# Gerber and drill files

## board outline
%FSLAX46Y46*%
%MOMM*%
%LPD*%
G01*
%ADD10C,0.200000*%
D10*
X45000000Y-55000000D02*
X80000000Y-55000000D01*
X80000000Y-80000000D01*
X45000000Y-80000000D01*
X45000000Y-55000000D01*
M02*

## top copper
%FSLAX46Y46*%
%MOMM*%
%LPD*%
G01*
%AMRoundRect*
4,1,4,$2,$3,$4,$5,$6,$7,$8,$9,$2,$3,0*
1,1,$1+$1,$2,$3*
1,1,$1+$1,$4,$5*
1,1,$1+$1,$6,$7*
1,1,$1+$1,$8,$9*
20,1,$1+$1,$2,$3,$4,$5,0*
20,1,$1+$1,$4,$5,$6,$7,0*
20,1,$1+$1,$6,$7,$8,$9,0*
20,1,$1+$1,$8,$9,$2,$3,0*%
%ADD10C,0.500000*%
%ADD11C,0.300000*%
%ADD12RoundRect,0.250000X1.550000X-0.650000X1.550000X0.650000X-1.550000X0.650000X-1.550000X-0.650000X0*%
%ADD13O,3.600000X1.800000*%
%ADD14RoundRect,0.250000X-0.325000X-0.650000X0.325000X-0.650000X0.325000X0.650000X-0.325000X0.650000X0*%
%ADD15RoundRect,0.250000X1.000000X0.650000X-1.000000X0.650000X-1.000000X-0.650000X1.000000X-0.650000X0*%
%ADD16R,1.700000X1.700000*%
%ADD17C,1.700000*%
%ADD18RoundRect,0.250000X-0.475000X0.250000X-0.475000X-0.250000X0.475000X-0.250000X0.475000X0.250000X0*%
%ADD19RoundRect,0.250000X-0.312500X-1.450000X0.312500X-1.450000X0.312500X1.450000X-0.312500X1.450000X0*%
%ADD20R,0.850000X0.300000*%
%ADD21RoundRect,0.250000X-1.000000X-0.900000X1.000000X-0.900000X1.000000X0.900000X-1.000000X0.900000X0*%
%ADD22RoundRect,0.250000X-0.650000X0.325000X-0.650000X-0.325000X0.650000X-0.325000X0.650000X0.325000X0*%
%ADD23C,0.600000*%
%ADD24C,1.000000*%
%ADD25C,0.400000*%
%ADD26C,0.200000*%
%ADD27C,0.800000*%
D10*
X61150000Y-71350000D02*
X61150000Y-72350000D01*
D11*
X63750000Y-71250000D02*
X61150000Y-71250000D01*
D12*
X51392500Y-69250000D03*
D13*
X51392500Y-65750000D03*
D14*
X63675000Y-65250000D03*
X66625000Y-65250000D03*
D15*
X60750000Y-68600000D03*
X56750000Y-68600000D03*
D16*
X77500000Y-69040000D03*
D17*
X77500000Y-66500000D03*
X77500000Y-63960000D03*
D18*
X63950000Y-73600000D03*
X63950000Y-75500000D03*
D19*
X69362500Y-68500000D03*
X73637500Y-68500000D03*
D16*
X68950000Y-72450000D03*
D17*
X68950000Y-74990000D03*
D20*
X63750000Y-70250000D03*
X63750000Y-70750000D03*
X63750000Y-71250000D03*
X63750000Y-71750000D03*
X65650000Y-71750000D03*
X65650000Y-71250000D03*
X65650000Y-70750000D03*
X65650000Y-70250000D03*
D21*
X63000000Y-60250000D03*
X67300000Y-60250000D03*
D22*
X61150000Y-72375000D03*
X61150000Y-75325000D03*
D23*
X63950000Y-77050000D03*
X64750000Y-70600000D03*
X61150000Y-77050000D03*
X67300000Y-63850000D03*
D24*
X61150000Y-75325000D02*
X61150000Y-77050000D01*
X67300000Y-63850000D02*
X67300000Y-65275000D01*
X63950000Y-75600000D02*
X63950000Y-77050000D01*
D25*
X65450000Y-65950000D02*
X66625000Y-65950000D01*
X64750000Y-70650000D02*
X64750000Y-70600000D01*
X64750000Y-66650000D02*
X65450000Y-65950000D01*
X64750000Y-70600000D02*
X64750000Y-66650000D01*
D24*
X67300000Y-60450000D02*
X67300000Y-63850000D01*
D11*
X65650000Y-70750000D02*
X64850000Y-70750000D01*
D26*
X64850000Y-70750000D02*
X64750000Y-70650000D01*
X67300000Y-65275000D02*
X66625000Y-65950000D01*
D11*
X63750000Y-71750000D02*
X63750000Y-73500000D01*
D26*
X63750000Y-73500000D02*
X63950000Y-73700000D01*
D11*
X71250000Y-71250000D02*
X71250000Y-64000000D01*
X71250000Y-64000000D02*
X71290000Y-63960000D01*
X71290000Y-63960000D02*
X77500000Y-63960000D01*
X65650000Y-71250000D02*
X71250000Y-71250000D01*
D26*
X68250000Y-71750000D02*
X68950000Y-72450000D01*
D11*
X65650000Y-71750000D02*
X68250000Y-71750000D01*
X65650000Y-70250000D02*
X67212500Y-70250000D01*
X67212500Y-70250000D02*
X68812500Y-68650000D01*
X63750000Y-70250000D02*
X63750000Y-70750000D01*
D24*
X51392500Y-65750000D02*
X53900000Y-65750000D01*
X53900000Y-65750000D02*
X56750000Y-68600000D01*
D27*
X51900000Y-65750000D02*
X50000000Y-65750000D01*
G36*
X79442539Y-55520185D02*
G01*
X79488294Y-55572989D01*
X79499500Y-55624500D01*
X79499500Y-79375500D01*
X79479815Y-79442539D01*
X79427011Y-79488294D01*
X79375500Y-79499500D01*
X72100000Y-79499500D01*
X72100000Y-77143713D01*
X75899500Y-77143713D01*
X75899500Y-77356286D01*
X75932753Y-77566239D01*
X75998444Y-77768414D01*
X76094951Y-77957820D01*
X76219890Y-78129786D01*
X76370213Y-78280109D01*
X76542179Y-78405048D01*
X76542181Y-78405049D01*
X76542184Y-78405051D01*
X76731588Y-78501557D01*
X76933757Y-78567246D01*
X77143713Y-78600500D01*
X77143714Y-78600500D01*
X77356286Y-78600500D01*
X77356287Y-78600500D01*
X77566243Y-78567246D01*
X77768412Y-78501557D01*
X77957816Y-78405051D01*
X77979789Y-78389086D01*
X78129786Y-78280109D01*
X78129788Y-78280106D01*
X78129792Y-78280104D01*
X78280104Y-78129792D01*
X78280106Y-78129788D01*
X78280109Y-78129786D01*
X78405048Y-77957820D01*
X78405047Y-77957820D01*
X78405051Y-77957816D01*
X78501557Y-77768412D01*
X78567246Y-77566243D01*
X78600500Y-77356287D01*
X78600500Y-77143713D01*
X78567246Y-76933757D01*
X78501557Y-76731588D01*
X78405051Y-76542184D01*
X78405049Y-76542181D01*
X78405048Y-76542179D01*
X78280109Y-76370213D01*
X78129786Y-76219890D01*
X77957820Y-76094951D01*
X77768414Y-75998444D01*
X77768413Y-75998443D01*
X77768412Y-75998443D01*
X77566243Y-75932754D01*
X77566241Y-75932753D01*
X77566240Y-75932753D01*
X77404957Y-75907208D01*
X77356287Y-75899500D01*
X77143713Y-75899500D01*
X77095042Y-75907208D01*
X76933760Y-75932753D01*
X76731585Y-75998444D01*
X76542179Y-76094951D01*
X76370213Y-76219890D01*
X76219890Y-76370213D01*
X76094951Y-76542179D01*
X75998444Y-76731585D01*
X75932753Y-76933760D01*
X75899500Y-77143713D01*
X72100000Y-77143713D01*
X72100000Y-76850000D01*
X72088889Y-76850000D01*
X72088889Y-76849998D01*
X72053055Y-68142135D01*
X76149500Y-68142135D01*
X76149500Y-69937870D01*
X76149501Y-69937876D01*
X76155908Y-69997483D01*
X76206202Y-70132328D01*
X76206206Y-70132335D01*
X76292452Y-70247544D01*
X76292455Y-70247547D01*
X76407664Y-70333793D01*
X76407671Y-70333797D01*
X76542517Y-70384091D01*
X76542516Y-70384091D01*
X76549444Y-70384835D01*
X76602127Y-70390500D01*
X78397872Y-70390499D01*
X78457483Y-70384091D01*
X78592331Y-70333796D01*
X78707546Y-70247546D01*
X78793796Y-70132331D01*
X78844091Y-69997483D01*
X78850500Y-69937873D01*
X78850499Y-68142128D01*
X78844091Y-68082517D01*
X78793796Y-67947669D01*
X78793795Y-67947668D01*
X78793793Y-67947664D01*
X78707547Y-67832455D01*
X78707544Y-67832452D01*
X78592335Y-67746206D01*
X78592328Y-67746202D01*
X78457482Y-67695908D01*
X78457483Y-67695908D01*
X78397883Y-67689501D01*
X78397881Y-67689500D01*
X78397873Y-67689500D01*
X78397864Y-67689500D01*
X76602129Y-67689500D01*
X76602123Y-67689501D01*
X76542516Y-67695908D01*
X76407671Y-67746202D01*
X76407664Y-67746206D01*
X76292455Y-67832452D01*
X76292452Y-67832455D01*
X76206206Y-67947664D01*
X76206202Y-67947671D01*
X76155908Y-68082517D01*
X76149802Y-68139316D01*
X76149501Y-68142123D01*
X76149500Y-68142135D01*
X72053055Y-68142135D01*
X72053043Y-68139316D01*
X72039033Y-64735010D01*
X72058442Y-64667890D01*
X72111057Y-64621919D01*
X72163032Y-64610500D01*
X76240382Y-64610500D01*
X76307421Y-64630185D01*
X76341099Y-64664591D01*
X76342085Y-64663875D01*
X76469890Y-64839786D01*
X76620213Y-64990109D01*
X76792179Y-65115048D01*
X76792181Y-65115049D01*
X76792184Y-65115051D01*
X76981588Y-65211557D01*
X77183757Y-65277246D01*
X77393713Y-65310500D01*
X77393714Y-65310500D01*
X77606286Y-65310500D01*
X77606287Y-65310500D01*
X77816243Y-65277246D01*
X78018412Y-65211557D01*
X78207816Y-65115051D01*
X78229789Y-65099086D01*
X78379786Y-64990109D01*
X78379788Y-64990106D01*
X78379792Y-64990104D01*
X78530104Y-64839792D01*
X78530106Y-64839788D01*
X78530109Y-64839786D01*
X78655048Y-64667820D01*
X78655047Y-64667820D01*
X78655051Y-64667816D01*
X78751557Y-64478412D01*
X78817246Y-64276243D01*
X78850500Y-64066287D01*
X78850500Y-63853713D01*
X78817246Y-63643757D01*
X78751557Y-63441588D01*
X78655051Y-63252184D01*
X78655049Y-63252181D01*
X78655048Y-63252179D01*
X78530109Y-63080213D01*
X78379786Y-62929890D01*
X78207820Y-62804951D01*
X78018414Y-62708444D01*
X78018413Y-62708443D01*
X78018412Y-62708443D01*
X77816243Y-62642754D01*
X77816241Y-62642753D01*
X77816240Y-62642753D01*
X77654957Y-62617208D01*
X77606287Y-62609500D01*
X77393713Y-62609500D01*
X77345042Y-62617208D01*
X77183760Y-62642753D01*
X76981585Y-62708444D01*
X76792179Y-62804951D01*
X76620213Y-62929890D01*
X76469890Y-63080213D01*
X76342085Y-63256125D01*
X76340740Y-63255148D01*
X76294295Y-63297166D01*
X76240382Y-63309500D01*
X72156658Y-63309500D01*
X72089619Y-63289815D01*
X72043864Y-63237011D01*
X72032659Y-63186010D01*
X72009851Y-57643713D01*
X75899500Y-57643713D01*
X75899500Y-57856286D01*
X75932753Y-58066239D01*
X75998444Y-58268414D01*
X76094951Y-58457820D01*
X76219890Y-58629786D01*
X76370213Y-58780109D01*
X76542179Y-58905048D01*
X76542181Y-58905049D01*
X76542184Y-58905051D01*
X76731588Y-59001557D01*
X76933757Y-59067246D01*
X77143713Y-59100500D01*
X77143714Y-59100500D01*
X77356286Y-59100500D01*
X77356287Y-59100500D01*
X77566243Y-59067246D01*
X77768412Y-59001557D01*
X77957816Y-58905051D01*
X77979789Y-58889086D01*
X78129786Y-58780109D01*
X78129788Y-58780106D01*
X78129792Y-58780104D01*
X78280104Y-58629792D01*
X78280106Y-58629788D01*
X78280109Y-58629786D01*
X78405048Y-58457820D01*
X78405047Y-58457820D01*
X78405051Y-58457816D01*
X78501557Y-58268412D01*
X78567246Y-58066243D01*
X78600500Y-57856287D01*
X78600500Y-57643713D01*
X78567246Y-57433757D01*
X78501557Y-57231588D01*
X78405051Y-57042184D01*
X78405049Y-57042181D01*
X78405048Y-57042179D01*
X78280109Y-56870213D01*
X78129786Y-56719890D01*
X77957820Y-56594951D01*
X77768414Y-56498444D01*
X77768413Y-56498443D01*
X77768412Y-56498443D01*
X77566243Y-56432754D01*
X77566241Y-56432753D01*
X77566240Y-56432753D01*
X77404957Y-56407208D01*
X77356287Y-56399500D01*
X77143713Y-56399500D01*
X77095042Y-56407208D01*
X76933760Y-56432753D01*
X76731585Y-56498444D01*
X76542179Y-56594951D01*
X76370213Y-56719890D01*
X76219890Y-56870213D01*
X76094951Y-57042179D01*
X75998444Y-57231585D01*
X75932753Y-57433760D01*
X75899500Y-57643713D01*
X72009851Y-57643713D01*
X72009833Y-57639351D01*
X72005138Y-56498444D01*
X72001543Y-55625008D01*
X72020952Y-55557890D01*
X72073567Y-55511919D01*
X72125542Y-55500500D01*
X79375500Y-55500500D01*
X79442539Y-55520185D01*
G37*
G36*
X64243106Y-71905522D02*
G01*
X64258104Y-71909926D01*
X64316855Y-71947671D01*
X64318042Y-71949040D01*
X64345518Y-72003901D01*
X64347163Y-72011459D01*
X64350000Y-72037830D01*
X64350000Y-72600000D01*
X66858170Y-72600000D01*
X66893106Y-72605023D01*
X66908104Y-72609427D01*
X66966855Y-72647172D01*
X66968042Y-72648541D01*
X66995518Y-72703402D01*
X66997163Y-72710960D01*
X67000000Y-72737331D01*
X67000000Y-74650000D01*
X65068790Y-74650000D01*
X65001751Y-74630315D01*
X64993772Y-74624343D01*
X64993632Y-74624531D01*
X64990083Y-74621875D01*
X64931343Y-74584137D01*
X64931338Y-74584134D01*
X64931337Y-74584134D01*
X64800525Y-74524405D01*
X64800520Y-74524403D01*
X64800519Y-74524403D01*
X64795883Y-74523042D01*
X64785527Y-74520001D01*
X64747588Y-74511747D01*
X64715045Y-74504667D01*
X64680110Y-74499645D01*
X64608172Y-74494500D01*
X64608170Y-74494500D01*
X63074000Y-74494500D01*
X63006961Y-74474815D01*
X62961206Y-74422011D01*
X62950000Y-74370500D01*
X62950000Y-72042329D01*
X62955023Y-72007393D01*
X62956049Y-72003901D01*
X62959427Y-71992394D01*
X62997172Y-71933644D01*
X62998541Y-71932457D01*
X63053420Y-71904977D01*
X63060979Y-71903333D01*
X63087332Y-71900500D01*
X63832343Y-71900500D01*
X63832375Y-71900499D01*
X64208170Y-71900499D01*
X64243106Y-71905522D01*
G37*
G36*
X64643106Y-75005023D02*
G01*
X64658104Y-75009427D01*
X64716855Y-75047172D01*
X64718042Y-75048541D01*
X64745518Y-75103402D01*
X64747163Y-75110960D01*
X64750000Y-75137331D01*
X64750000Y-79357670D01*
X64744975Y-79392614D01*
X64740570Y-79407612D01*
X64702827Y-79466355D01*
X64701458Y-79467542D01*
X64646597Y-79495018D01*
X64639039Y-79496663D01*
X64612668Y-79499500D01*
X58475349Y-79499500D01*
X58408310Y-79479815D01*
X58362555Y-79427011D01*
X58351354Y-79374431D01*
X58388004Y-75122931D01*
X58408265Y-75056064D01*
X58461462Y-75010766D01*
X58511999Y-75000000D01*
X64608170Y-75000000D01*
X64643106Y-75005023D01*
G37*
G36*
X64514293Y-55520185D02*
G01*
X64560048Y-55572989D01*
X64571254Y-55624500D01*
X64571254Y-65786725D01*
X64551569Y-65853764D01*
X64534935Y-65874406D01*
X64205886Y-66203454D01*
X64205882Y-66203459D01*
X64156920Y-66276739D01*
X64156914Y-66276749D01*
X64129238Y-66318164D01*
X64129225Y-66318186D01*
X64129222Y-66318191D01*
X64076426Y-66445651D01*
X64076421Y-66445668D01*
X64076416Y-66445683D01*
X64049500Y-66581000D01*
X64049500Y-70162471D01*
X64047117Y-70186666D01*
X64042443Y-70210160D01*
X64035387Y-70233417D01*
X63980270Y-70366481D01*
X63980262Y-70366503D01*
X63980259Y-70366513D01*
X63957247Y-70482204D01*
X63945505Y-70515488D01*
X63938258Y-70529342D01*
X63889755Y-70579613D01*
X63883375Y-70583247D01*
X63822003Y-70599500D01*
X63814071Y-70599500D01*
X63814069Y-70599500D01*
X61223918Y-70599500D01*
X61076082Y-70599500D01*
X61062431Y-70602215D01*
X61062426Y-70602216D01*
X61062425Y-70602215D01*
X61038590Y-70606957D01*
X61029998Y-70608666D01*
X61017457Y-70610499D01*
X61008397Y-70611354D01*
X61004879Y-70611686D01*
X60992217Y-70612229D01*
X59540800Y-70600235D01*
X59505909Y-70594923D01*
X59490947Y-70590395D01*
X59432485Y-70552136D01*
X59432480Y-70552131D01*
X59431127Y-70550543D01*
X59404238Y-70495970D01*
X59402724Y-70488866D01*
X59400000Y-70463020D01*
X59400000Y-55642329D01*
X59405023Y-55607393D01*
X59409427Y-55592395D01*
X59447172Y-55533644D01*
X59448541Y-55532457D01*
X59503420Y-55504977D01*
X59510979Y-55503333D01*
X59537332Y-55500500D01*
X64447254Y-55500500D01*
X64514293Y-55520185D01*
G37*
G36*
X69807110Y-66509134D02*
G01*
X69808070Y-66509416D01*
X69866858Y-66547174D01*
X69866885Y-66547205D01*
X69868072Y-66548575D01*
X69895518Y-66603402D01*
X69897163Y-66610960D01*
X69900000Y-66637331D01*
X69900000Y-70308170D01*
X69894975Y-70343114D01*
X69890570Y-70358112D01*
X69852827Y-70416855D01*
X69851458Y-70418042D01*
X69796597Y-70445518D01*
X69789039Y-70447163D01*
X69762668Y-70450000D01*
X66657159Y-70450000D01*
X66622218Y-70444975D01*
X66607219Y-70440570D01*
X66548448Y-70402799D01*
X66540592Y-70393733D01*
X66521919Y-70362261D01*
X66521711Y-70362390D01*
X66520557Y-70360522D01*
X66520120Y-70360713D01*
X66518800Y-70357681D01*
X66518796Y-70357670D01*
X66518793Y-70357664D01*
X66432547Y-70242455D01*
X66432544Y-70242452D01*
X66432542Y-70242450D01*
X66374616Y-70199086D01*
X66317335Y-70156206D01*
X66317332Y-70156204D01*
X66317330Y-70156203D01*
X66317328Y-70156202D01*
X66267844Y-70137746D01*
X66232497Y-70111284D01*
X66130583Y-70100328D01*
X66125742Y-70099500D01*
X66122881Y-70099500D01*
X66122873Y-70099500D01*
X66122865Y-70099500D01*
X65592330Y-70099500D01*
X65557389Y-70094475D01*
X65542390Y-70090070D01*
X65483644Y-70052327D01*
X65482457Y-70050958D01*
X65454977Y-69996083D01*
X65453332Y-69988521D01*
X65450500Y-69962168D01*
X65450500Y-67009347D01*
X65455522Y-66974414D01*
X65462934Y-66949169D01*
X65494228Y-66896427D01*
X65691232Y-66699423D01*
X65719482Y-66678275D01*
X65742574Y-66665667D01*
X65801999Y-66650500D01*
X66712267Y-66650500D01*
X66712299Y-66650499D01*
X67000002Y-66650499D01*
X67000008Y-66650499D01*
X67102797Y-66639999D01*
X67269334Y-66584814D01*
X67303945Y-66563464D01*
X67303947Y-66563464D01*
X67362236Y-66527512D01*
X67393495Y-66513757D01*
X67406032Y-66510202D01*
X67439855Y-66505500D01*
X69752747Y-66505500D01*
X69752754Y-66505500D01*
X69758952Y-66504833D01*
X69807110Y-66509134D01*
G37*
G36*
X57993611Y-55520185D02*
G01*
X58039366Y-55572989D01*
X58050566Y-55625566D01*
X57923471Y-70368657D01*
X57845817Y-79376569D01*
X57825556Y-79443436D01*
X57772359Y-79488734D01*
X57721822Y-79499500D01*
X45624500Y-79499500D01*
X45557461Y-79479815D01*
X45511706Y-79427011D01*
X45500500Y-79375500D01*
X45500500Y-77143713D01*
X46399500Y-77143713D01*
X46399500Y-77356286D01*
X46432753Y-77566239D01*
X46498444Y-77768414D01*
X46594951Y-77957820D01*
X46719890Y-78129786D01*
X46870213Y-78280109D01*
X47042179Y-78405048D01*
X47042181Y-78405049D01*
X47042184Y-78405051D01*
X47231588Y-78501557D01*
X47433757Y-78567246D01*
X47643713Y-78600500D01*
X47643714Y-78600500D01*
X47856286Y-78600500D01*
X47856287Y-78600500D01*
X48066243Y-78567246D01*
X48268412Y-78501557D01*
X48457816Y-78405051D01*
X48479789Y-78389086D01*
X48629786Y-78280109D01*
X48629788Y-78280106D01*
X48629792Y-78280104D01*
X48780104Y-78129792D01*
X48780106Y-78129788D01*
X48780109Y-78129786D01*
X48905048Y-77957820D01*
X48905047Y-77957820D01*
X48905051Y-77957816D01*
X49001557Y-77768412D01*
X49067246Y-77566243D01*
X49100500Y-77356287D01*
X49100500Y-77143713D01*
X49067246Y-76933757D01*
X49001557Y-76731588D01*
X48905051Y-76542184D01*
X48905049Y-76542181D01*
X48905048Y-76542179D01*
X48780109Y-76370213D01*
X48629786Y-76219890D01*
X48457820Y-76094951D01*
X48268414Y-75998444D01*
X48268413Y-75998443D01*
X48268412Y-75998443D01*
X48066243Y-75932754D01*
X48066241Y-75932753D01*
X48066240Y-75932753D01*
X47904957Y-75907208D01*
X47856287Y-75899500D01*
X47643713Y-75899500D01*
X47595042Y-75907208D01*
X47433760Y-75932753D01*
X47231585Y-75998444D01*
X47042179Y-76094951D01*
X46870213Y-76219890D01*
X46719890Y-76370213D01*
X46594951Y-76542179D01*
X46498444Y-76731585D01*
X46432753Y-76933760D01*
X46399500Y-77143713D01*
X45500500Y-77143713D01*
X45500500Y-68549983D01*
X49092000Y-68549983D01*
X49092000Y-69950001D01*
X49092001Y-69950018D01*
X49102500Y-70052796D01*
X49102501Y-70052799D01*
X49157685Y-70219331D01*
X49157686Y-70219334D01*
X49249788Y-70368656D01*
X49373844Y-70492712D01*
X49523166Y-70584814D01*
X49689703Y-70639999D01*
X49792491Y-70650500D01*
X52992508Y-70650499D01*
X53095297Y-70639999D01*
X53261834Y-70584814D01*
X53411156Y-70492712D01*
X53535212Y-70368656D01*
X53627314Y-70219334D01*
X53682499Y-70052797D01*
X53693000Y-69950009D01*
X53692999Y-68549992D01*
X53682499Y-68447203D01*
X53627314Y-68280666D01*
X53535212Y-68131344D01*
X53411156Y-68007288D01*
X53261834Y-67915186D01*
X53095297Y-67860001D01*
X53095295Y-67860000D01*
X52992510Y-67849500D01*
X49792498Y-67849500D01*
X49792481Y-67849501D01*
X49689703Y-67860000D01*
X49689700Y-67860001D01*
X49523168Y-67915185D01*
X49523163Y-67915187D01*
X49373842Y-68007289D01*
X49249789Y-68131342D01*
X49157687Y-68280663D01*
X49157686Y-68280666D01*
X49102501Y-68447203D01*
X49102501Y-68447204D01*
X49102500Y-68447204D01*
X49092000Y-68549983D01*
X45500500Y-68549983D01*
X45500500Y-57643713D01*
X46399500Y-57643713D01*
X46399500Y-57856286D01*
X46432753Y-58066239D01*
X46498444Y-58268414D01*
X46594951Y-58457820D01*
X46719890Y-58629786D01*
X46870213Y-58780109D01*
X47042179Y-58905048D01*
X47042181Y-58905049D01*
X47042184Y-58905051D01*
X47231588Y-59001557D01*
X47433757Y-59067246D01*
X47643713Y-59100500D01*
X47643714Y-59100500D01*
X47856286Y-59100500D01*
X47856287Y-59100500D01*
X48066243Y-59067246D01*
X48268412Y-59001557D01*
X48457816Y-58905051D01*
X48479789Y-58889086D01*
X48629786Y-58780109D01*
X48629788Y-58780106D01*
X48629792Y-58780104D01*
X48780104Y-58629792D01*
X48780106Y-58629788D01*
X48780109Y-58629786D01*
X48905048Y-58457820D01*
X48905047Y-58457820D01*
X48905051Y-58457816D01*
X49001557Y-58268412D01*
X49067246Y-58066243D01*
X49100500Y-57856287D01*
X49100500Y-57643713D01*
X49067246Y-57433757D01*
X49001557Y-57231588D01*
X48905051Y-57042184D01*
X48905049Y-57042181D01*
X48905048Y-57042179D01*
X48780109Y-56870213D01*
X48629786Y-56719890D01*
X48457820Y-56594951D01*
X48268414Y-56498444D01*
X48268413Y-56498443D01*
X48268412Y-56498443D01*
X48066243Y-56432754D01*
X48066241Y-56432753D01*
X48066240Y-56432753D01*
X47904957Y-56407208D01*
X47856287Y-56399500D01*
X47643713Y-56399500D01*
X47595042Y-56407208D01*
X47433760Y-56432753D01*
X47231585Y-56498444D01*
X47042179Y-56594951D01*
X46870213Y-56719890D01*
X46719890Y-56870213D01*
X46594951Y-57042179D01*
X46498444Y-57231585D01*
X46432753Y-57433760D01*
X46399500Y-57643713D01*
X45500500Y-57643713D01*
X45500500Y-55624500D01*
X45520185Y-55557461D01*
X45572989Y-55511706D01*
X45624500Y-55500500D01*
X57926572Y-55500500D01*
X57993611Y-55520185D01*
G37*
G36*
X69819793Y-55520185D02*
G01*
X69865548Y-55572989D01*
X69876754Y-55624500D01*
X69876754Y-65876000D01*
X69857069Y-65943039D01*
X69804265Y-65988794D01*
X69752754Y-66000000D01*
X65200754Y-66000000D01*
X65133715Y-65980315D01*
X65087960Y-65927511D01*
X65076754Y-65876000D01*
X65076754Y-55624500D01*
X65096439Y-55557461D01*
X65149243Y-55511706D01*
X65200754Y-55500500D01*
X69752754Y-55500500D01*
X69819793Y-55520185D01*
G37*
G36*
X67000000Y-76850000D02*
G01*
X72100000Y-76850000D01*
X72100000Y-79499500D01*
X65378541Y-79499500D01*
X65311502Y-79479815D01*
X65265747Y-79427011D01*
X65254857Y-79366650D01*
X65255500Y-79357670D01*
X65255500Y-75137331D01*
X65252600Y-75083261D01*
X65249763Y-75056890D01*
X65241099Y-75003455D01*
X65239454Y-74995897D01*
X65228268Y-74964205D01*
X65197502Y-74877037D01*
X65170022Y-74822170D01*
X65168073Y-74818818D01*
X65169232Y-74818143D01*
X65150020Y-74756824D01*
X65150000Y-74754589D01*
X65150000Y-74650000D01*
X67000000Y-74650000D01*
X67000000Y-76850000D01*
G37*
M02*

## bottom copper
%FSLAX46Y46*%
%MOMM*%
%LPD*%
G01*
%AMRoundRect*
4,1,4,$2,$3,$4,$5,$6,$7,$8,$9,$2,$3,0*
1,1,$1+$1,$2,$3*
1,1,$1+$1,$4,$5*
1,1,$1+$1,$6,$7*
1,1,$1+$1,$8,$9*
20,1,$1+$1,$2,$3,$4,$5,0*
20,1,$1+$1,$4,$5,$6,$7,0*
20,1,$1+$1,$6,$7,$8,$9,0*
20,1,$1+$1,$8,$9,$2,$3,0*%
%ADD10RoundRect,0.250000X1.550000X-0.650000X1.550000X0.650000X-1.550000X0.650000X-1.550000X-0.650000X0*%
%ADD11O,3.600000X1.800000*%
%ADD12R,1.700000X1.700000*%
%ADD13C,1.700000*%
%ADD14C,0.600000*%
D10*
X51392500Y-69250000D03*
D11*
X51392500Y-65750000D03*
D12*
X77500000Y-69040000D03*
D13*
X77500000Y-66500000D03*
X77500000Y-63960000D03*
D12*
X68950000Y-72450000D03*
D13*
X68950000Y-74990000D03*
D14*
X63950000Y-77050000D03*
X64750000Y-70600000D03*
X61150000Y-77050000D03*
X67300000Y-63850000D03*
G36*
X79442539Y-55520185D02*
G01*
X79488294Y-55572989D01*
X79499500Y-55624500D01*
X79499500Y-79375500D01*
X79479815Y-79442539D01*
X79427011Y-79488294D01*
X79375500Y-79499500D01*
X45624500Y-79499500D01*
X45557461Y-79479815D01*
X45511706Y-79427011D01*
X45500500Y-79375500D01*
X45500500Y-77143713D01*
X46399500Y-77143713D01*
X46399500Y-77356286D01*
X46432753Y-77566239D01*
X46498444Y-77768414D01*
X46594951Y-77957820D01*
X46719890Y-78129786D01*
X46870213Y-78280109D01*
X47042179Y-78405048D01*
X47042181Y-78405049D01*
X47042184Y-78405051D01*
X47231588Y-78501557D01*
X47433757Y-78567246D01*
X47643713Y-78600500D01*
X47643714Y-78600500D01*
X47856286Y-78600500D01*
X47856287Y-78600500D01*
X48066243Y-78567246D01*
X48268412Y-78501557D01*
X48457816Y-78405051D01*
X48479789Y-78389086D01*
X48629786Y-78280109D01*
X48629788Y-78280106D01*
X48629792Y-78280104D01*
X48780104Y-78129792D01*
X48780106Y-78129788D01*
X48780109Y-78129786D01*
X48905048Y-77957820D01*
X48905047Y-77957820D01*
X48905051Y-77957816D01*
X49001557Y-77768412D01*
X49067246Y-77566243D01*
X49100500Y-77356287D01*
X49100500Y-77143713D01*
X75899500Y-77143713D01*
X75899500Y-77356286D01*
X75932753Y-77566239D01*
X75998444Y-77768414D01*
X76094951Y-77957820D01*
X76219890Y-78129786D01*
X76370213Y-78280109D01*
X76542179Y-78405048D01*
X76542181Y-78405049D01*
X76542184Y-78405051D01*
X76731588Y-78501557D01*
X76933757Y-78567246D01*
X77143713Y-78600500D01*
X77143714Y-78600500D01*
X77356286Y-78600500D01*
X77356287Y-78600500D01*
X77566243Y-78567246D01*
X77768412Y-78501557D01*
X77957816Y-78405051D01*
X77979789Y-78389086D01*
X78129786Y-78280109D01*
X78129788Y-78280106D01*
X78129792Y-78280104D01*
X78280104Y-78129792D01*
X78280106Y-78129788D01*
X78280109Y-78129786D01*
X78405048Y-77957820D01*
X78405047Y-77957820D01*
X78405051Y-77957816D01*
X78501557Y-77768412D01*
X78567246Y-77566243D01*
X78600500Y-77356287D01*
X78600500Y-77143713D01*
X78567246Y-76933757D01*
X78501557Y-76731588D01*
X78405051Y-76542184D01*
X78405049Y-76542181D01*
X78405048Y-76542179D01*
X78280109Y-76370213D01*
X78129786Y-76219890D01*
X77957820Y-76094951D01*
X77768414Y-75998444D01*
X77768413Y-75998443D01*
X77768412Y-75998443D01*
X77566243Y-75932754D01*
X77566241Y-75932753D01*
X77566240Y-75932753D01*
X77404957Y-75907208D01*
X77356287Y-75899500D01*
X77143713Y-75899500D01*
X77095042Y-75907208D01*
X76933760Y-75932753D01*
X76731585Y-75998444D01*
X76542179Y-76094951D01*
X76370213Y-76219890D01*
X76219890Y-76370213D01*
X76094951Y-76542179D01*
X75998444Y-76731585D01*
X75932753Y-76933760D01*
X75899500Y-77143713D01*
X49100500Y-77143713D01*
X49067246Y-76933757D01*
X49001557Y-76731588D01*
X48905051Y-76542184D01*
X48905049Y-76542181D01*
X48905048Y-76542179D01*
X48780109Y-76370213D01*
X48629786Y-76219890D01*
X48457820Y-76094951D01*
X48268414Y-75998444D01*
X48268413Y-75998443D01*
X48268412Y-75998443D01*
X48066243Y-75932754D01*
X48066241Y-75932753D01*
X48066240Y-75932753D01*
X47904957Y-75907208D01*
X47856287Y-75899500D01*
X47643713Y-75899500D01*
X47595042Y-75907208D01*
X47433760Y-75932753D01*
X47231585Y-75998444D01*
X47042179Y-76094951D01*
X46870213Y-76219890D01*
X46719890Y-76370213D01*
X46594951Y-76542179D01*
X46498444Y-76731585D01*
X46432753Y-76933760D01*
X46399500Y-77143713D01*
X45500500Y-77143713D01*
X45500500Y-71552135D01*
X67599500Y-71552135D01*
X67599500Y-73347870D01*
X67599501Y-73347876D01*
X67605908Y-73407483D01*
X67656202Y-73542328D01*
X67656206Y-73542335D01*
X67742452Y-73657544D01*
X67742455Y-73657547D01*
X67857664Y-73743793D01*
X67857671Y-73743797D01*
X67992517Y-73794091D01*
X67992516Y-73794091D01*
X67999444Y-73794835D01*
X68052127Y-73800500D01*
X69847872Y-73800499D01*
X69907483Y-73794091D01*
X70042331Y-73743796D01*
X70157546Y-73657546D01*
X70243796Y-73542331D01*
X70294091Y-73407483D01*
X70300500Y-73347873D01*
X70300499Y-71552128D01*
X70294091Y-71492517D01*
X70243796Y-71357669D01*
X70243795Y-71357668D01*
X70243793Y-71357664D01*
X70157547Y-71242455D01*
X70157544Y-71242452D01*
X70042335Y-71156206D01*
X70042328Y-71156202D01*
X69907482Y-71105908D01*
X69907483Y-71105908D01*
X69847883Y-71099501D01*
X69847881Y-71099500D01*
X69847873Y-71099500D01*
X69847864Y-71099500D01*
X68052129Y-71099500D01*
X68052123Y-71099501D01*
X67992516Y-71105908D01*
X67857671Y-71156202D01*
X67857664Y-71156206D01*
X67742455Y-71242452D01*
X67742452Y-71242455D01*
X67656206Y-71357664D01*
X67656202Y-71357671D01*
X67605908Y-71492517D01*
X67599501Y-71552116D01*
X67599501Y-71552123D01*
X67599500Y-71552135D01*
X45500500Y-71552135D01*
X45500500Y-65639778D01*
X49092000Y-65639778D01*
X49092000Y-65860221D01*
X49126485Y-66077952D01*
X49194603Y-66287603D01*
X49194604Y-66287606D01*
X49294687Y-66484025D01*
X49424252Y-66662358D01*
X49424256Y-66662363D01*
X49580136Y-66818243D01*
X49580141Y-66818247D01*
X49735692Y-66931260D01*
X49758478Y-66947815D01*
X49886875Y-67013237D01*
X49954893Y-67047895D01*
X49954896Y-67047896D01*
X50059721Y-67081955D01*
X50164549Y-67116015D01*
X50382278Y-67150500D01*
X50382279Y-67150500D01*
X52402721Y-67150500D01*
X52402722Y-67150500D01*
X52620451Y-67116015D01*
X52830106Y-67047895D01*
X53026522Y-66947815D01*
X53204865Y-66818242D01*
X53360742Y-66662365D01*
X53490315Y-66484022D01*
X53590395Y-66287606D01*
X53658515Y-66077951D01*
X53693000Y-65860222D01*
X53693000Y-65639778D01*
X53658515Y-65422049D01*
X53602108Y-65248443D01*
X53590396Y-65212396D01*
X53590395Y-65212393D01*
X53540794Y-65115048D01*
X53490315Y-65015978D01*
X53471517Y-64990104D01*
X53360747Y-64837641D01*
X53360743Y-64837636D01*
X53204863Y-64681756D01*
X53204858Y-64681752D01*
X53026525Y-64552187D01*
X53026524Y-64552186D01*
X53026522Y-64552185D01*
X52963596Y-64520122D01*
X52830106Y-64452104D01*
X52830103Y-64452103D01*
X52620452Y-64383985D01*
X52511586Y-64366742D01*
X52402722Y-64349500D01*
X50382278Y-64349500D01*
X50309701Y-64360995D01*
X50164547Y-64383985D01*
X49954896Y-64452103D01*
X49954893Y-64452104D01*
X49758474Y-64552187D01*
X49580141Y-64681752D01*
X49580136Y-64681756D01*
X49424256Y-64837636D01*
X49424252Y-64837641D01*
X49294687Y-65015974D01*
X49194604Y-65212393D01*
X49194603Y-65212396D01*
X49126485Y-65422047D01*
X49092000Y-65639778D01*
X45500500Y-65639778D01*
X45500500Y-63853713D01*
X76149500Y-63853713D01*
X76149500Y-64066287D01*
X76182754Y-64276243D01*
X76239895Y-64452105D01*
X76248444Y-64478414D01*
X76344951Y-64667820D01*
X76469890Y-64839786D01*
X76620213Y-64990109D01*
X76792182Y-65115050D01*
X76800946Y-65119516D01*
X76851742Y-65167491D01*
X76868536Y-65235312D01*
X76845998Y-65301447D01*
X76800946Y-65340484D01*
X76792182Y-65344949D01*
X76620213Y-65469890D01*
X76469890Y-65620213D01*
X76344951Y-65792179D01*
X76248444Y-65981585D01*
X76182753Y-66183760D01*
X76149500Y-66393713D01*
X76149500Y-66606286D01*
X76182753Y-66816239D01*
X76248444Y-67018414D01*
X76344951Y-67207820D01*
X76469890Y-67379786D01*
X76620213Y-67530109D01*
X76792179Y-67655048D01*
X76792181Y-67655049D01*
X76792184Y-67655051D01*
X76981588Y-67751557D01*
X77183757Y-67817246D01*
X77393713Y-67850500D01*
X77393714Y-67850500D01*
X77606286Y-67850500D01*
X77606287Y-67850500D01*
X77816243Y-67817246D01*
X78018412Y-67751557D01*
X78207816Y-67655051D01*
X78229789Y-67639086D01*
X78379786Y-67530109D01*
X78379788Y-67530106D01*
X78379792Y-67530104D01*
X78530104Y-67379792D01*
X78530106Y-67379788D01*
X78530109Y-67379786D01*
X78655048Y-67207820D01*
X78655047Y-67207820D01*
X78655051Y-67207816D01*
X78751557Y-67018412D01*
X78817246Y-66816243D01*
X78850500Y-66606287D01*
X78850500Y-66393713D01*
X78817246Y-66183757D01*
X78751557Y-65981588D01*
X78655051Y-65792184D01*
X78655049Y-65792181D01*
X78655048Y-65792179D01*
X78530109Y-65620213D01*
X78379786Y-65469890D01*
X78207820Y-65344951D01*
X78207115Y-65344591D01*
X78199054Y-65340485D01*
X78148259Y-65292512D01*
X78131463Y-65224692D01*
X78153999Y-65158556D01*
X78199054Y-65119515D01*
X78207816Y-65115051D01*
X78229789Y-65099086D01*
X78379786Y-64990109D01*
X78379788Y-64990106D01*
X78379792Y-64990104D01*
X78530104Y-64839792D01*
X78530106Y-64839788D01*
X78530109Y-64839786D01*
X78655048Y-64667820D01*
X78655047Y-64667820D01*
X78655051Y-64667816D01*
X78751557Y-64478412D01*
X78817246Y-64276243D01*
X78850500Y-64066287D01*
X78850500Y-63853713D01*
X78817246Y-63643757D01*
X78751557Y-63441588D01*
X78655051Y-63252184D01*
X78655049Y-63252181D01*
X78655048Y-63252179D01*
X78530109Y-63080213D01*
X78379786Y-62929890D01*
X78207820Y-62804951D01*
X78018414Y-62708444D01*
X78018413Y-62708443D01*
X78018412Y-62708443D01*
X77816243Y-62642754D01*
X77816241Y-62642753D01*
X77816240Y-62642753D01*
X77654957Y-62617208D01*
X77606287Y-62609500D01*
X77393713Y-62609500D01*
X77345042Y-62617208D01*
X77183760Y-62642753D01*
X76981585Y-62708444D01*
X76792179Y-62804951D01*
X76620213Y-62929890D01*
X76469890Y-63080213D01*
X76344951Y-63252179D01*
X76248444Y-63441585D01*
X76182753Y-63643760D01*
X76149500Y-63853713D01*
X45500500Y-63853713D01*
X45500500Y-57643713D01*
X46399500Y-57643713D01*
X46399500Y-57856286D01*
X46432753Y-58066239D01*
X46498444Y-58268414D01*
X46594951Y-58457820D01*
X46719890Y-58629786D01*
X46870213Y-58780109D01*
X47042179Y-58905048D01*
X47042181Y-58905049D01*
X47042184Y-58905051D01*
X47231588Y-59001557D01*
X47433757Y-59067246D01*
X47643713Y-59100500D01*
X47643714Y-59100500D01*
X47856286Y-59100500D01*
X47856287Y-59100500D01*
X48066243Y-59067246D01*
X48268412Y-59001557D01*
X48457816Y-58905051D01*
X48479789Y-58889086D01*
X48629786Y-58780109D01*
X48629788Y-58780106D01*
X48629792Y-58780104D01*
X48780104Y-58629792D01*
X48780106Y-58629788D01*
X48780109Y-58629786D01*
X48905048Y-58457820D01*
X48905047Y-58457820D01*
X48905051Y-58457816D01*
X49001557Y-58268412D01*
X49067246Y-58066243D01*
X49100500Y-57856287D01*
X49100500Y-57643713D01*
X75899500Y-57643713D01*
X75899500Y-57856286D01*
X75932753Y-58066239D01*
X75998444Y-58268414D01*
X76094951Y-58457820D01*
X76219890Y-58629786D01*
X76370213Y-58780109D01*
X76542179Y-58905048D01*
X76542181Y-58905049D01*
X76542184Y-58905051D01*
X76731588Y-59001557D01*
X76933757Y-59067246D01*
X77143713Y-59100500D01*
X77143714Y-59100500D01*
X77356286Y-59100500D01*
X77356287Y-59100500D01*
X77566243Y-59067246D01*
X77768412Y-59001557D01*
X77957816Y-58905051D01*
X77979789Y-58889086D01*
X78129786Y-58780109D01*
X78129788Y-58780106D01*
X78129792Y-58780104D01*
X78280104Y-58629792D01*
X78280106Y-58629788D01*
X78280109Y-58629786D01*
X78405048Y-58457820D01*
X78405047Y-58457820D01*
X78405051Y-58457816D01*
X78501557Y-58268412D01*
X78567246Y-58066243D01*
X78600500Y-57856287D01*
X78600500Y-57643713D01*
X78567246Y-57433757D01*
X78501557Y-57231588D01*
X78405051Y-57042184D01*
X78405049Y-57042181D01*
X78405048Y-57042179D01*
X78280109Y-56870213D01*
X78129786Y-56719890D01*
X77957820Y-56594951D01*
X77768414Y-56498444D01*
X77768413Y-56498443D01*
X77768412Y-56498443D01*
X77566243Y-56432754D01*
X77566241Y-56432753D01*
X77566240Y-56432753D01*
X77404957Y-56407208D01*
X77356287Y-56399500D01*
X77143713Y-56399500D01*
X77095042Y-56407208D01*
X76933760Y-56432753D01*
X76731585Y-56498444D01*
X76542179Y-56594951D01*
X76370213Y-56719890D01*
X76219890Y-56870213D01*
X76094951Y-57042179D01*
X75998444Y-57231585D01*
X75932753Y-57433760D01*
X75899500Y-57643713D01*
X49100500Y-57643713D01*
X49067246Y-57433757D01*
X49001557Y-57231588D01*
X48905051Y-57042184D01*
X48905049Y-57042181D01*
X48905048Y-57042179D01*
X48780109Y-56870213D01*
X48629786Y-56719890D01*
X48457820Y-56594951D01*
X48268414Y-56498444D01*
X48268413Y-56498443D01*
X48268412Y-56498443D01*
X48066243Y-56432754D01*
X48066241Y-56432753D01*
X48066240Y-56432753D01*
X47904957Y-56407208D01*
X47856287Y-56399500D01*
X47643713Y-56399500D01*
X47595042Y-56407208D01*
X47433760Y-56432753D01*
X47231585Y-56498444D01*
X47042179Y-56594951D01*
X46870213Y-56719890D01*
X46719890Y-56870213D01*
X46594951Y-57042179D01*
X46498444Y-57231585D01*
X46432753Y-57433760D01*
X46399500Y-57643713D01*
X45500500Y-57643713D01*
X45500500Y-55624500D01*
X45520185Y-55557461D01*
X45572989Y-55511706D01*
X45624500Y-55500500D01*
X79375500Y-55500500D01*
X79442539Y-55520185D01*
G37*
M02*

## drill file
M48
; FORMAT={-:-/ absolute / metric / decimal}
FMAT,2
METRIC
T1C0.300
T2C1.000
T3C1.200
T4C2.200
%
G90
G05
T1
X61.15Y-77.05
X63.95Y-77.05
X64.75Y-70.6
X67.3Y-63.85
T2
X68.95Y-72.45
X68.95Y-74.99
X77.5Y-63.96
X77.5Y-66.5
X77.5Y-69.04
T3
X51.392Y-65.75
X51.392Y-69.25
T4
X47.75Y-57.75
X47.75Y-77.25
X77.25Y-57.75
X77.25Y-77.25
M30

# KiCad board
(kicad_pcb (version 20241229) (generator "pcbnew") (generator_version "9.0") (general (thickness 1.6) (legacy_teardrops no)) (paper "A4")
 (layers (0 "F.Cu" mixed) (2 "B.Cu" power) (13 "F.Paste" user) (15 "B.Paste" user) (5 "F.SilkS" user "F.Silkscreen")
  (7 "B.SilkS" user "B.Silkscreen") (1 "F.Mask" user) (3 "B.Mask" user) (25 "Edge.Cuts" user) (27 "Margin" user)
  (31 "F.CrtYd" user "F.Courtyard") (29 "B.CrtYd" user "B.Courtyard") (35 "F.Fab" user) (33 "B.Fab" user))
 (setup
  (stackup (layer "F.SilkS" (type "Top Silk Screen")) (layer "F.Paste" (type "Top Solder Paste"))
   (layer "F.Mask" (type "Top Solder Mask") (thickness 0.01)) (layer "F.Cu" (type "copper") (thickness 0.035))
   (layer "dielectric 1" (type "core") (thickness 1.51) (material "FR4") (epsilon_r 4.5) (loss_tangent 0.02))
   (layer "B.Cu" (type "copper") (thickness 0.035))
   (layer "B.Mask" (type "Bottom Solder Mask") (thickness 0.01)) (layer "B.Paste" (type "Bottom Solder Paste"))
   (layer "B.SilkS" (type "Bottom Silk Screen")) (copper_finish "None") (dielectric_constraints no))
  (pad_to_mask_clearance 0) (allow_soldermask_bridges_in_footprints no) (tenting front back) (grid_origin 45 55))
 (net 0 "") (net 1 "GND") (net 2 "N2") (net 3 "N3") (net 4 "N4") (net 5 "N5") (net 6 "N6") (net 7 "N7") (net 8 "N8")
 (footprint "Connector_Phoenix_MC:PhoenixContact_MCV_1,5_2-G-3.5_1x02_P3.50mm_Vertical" (layer "F.Cu") (at 51.3925 69.25 90)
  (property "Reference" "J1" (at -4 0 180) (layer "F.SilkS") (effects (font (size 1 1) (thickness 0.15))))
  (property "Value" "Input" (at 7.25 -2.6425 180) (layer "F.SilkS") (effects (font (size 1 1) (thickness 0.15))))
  (pad "1" thru_hole roundrect (at 0 0 90) (size 1.8 3.6) (drill 1.2) (layers "*.Cu" "*.Mask") (remove_unused_layers no)
   (roundrect_rratio 0.138889) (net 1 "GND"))
  (pad "2" thru_hole oval (at 3.5 0 90) (size 1.8 3.6) (drill 1.2) (layers "*.Cu" "*.Mask") (remove_unused_layers no) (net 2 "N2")))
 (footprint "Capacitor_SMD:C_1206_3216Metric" (layer "F.Cu") (at 65.15 65.25)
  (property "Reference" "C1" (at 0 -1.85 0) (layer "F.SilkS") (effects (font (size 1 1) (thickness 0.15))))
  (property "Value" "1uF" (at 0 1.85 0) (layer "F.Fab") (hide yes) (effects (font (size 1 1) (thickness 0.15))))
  (pad "1" smd roundrect (at -1.475 0) (size 1.15 1.8) (layers "F.Cu" "F.Mask" "F.Paste") (roundrect_rratio 0.217391) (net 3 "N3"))
  (pad "2" smd roundrect (at 1.475 0) (size 1.15 1.8) (layers "F.Cu" "F.Mask" "F.Paste") (roundrect_rratio 0.217391) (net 1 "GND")))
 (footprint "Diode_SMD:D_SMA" (layer "F.Cu") (at 58.75 68.6 180)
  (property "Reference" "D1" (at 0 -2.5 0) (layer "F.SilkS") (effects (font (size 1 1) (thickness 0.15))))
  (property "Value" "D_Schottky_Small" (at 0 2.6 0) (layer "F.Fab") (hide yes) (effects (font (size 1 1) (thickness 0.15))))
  (pad "1" smd roundrect (at -2 0 180) (size 2.5 1.8) (layers "F.Cu" "F.Mask" "F.Paste") (roundrect_rratio 0.1388888889) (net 3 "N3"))
  (pad "2" smd roundrect (at 2 0 180) (size 2.5 1.8) (layers "F.Cu" "F.Mask" "F.Paste") (roundrect_rratio 0.1388888889) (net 2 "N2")))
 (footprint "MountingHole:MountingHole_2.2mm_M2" (layer "F.Cu") (at 47.75 77.25)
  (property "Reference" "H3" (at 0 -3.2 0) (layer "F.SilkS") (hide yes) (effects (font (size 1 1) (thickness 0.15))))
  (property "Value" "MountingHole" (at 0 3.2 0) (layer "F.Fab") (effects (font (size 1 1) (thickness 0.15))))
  (pad "" np_thru_hole circle (at 0 0) (size 2.2 2.2) (drill 2.2) (layers "*.Cu" "*.Mask")))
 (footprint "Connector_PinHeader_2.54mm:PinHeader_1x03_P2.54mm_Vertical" (layer "F.Cu") (at 77.5 69.04 180)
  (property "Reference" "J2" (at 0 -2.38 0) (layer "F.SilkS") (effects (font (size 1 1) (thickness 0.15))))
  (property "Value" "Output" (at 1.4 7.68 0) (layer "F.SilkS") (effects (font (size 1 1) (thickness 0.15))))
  (pad "1" thru_hole rect (at 0 0 180) (size 1.7 1.7) (drill 1) (layers "*.Cu" "*.Mask") (remove_unused_layers no) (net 1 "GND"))
  (pad "2" thru_hole circle (at 0 2.54 180) (size 1.7 1.7) (drill 1) (layers "*.Cu" "*.Mask") (remove_unused_layers no) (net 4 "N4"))
  (pad "3" thru_hole circle (at 0 5.08 180) (size 1.7 1.7) (drill 1) (layers "*.Cu" "*.Mask") (remove_unused_layers no) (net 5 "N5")))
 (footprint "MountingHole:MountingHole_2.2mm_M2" (layer "F.Cu") (at 77.25 77.25)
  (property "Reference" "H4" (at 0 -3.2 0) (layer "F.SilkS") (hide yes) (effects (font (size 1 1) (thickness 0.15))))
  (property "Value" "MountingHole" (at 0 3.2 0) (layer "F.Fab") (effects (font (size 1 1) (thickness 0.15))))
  (pad "" np_thru_hole circle (at 0 0) (size 2.2 2.2) (drill 2.2) (layers "*.Cu" "*.Mask")))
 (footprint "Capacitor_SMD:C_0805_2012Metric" (layer "F.Cu") (at 63.95 74.55 -90)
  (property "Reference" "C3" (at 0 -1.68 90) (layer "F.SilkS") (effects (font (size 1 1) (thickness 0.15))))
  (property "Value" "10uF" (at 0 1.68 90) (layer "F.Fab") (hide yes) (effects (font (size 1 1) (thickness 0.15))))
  (pad "1" smd roundrect (at -0.95 0 270) (size 1 1.45) (layers "F.Cu" "F.Mask" "F.Paste") (roundrect_rratio 0.25) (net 4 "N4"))
  (pad "2" smd roundrect (at 0.95 0 270) (size 1 1.45) (layers "F.Cu" "F.Mask" "F.Paste") (roundrect_rratio 0.25) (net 1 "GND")))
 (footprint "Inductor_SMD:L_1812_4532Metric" (layer "F.Cu") (at 71.5 68.5)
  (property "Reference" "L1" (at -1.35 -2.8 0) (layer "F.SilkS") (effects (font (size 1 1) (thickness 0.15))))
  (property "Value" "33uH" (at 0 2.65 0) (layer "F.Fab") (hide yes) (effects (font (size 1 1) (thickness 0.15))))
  (pad "1" smd roundrect (at -2.1375 0) (size 1.125 3.4) (layers "F.Cu" "F.Mask" "F.Paste") (roundrect_rratio 0.222222) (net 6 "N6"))
  (pad "2" smd roundrect (at 2.1375 0) (size 1.125 3.4) (layers "F.Cu" "F.Mask" "F.Paste") (roundrect_rratio 0.222222) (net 4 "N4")))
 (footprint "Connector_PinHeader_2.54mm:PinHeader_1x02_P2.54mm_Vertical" (layer "F.Cu") (at 68.95 72.45)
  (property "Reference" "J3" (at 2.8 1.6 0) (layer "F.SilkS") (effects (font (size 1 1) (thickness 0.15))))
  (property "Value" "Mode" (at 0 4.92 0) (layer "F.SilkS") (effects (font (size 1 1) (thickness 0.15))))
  (pad "1" thru_hole rect (at 0 0) (size 1.7 1.7) (drill 1) (layers "*.Cu" "*.Mask") (remove_unused_layers no) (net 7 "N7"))
  (pad "2" thru_hole circle (at 0 2.54) (size 1.7 1.7) (drill 1) (layers "*.Cu" "*.Mask") (remove_unused_layers no) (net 1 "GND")))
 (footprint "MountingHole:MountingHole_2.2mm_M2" (layer "F.Cu") (at 47.75 57.75)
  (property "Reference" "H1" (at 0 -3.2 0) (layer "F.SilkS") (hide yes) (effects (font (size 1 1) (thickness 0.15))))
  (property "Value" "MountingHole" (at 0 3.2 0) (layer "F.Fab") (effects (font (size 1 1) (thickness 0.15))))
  (pad "" np_thru_hole circle (at 0 0) (size 2.2 2.2) (drill 2.2) (layers "*.Cu" "*.Mask")))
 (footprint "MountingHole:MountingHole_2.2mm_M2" (layer "F.Cu") (at 77.25 57.75)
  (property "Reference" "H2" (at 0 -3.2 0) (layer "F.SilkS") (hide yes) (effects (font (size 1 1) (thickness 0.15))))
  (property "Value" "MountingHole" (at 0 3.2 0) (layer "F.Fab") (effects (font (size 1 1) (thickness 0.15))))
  (pad "" np_thru_hole circle (at 0 0) (size 2.2 2.2) (drill 2.2) (layers "*.Cu" "*.Mask")))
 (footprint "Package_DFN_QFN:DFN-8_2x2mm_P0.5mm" (layer "F.Cu") (at 64.7 71)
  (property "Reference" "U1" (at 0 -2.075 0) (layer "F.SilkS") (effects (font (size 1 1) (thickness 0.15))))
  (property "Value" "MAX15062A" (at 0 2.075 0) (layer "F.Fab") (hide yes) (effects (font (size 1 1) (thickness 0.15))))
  (pad "1" smd rect (at -0.95 -0.75) (size 0.85 0.3) (layers "F.Cu" "F.Mask" "F.Paste") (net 3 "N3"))
  (pad "2" smd rect (at -0.95 -0.25) (size 0.85 0.3) (layers "F.Cu" "F.Mask" "F.Paste") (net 3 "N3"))
  (pad "3" smd rect (at -0.95 0.25) (size 0.85 0.3) (layers "F.Cu" "F.Mask" "F.Paste") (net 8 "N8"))
  (pad "4" smd rect (at -0.95 0.75) (size 0.85 0.3) (layers "F.Cu" "F.Mask" "F.Paste") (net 4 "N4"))
  (pad "5" smd rect (at 0.95 0.75) (size 0.85 0.3) (layers "F.Cu" "F.Mask" "F.Paste") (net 7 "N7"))
  (pad "6" smd rect (at 0.95 0.25) (size 0.85 0.3) (layers "F.Cu" "F.Mask" "F.Paste") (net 5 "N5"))
  (pad "7" smd rect (at 0.95 -0.25) (size 0.85 0.3) (layers "F.Cu" "F.Mask" "F.Paste") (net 1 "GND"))
  (pad "8" smd rect (at 0.95 -0.75) (size 0.85 0.3) (layers "F.Cu" "F.Mask" "F.Paste") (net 6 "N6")))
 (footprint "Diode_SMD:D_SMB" (layer "F.Cu") (at 65.15 60.25)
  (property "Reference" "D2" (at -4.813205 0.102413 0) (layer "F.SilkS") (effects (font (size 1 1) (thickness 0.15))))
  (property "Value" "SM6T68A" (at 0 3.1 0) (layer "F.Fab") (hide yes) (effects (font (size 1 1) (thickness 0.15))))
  (pad "1" smd roundrect (at -2.15 0) (size 2.5 2.3) (layers "F.Cu" "F.Mask" "F.Paste") (roundrect_rratio 0.1086956522) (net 3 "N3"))
  (pad "2" smd roundrect (at 2.15 0) (size 2.5 2.3) (layers "F.Cu" "F.Mask" "F.Paste") (roundrect_rratio 0.1086956522) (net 1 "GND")))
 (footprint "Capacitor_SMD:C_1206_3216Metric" (layer "F.Cu") (at 61.15 73.85 -90)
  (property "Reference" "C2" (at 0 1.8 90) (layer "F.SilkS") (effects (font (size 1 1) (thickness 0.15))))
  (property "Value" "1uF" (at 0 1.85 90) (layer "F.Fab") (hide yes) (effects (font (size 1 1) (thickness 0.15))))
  (pad "1" smd roundrect (at -1.475 0 270) (size 1.15 1.8) (layers "F.Cu" "F.Mask" "F.Paste") (roundrect_rratio 0.217391) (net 8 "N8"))
  (pad "2" smd roundrect (at 1.475 0 270) (size 1.15 1.8) (layers "F.Cu" "F.Mask" "F.Paste") (roundrect_rratio 0.217391) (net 1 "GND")))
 (gr_line (start 61.15 71.35) (end 61.15 72.35) (stroke (width 0.5) (type solid)) (layer "F.Cu") (net 8))
 (gr_line (start 63.75 71.25) (end 61.15 71.25) (stroke (width 0.3) (type solid)) (layer "F.Cu") (net 8))
 (gr_rect (start 45 55) (end 80 80) (stroke (width 0.2) (type solid)) (fill no) (layer "Edge.Cuts"))
 (segment (start 61.15 75.325) (end 61.15 77.05) (width 1) (layer "F.Cu") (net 1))
 (segment (start 67.3 63.85) (end 67.3 65.275) (width 1) (layer "F.Cu") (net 1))
 (segment (start 63.95 75.6) (end 63.95 77.05) (width 1) (layer "F.Cu") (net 1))
 (segment (start 65.45 65.95) (end 66.625 65.95) (width 0.4) (layer "F.Cu") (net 1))
 (segment (start 64.75 70.65) (end 64.75 70.6) (width 0.4) (layer "F.Cu") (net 1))
 (segment (start 64.75 66.65) (end 65.45 65.95) (width 0.4) (layer "F.Cu") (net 1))
 (segment (start 64.75 70.6) (end 64.75 66.65) (width 0.4) (layer "F.Cu") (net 1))
 (segment (start 67.3 60.45) (end 67.3 63.85) (width 1) (layer "F.Cu") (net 1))
 (segment (start 65.65 70.75) (end 64.85 70.75) (width 0.3) (layer "F.Cu") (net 1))
 (segment (start 64.85 70.75) (end 64.75 70.65) (width 0.2) (layer "F.Cu") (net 1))
 (segment (start 67.3 65.275) (end 66.625 65.95) (width 0.2) (layer "F.Cu") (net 1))
 (via (at 63.95 77.05) (size 0.6) (drill 0.3) (layers "F.Cu" "B.Cu") (free yes) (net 1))
 (via (at 64.75 70.6) (size 0.6) (drill 0.3) (layers "F.Cu" "B.Cu") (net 1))
 (via (at 61.15 77.05) (size 0.6) (drill 0.3) (layers "F.Cu" "B.Cu") (free yes) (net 1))
 (via (at 67.3 63.85) (size 0.6) (drill 0.3) (layers "F.Cu" "B.Cu") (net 1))
 (segment (start 63.75 71.75) (end 63.75 73.5) (width 0.3) (layer "F.Cu") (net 4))
 (segment (start 63.75 73.5) (end 63.95 73.7) (width 0.2) (layer "F.Cu") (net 4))
 (segment (start 71.25 71.25) (end 71.25 64) (width 0.3) (layer "F.Cu") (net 5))
 (segment (start 71.25 64) (end 71.29 63.96) (width 0.3) (layer "F.Cu") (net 5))
 (segment (start 71.29 63.96) (end 77.5 63.96) (width 0.3) (layer "F.Cu") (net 5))
 (segment (start 65.65 71.25) (end 71.25 71.25) (width 0.3) (layer "F.Cu") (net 5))
 (segment (start 68.25 71.75) (end 68.95 72.45) (width 0.2) (layer "F.Cu") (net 7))
 (segment (start 65.65 71.75) (end 68.25 71.75) (width 0.3) (layer "F.Cu") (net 7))
 (segment (start 65.65 70.25) (end 67.2125 70.25) (width 0.3) (layer "F.Cu") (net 6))
 (segment (start 67.2125 70.25) (end 68.8125 68.65) (width 0.3) (layer "F.Cu") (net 6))
 (segment (start 63.75 70.25) (end 63.75 70.75) (width 0.3) (layer "F.Cu") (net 3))
 (segment (start 51.3925 65.75) (end 53.9 65.75) (width 1) (layer "F.Cu") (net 2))
 (segment (start 53.9 65.75) (end 56.75 68.6) (width 1) (layer "F.Cu") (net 2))
 (segment (start 51.9 65.75) (end 50 65.75) (width 0.8) (layer "F.Cu") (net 2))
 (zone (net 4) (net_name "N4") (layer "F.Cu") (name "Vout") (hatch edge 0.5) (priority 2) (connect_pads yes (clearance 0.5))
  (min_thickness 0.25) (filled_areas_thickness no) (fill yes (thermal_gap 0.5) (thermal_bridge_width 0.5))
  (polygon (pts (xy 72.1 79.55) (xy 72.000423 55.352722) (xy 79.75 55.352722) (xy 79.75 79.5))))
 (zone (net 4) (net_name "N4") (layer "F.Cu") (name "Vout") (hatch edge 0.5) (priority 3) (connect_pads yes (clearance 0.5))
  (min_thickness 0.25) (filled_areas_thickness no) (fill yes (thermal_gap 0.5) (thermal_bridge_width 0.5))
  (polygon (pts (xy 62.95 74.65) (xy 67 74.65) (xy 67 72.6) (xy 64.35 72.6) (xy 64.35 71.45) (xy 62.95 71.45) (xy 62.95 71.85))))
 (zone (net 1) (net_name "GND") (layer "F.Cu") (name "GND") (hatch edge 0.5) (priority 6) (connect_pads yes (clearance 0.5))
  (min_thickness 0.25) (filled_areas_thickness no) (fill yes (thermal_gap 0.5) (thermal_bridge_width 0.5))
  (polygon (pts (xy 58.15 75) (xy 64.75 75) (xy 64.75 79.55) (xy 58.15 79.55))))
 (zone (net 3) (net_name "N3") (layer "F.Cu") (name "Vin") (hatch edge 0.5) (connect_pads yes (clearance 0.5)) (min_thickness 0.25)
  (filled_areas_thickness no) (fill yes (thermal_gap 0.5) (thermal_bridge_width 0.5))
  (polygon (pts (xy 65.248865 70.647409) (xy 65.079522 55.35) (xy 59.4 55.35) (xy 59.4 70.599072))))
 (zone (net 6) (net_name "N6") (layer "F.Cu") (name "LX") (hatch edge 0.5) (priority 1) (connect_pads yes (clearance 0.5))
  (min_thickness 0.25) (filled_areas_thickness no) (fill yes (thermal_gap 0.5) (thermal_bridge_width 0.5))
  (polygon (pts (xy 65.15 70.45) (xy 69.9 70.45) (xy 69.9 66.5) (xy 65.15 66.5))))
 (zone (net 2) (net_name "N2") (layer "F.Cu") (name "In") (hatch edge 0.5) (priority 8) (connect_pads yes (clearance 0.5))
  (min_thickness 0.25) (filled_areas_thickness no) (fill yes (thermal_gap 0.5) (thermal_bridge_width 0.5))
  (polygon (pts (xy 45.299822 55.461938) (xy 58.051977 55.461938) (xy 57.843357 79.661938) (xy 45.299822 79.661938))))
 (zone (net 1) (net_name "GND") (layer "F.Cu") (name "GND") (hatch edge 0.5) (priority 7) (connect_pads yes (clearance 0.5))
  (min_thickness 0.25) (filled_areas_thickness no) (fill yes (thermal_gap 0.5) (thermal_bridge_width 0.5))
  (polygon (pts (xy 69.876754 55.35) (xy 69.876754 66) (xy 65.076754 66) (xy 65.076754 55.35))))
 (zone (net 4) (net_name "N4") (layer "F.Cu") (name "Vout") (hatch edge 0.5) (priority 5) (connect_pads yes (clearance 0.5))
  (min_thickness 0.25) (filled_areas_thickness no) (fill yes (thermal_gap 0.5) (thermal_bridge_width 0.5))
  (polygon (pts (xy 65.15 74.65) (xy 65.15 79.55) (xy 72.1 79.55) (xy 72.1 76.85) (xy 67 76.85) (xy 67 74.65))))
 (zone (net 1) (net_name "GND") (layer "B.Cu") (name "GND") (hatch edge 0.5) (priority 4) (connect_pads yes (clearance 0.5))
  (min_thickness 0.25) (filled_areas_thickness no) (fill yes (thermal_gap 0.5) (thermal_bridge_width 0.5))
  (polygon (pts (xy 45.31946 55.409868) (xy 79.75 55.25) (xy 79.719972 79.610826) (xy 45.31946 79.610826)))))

